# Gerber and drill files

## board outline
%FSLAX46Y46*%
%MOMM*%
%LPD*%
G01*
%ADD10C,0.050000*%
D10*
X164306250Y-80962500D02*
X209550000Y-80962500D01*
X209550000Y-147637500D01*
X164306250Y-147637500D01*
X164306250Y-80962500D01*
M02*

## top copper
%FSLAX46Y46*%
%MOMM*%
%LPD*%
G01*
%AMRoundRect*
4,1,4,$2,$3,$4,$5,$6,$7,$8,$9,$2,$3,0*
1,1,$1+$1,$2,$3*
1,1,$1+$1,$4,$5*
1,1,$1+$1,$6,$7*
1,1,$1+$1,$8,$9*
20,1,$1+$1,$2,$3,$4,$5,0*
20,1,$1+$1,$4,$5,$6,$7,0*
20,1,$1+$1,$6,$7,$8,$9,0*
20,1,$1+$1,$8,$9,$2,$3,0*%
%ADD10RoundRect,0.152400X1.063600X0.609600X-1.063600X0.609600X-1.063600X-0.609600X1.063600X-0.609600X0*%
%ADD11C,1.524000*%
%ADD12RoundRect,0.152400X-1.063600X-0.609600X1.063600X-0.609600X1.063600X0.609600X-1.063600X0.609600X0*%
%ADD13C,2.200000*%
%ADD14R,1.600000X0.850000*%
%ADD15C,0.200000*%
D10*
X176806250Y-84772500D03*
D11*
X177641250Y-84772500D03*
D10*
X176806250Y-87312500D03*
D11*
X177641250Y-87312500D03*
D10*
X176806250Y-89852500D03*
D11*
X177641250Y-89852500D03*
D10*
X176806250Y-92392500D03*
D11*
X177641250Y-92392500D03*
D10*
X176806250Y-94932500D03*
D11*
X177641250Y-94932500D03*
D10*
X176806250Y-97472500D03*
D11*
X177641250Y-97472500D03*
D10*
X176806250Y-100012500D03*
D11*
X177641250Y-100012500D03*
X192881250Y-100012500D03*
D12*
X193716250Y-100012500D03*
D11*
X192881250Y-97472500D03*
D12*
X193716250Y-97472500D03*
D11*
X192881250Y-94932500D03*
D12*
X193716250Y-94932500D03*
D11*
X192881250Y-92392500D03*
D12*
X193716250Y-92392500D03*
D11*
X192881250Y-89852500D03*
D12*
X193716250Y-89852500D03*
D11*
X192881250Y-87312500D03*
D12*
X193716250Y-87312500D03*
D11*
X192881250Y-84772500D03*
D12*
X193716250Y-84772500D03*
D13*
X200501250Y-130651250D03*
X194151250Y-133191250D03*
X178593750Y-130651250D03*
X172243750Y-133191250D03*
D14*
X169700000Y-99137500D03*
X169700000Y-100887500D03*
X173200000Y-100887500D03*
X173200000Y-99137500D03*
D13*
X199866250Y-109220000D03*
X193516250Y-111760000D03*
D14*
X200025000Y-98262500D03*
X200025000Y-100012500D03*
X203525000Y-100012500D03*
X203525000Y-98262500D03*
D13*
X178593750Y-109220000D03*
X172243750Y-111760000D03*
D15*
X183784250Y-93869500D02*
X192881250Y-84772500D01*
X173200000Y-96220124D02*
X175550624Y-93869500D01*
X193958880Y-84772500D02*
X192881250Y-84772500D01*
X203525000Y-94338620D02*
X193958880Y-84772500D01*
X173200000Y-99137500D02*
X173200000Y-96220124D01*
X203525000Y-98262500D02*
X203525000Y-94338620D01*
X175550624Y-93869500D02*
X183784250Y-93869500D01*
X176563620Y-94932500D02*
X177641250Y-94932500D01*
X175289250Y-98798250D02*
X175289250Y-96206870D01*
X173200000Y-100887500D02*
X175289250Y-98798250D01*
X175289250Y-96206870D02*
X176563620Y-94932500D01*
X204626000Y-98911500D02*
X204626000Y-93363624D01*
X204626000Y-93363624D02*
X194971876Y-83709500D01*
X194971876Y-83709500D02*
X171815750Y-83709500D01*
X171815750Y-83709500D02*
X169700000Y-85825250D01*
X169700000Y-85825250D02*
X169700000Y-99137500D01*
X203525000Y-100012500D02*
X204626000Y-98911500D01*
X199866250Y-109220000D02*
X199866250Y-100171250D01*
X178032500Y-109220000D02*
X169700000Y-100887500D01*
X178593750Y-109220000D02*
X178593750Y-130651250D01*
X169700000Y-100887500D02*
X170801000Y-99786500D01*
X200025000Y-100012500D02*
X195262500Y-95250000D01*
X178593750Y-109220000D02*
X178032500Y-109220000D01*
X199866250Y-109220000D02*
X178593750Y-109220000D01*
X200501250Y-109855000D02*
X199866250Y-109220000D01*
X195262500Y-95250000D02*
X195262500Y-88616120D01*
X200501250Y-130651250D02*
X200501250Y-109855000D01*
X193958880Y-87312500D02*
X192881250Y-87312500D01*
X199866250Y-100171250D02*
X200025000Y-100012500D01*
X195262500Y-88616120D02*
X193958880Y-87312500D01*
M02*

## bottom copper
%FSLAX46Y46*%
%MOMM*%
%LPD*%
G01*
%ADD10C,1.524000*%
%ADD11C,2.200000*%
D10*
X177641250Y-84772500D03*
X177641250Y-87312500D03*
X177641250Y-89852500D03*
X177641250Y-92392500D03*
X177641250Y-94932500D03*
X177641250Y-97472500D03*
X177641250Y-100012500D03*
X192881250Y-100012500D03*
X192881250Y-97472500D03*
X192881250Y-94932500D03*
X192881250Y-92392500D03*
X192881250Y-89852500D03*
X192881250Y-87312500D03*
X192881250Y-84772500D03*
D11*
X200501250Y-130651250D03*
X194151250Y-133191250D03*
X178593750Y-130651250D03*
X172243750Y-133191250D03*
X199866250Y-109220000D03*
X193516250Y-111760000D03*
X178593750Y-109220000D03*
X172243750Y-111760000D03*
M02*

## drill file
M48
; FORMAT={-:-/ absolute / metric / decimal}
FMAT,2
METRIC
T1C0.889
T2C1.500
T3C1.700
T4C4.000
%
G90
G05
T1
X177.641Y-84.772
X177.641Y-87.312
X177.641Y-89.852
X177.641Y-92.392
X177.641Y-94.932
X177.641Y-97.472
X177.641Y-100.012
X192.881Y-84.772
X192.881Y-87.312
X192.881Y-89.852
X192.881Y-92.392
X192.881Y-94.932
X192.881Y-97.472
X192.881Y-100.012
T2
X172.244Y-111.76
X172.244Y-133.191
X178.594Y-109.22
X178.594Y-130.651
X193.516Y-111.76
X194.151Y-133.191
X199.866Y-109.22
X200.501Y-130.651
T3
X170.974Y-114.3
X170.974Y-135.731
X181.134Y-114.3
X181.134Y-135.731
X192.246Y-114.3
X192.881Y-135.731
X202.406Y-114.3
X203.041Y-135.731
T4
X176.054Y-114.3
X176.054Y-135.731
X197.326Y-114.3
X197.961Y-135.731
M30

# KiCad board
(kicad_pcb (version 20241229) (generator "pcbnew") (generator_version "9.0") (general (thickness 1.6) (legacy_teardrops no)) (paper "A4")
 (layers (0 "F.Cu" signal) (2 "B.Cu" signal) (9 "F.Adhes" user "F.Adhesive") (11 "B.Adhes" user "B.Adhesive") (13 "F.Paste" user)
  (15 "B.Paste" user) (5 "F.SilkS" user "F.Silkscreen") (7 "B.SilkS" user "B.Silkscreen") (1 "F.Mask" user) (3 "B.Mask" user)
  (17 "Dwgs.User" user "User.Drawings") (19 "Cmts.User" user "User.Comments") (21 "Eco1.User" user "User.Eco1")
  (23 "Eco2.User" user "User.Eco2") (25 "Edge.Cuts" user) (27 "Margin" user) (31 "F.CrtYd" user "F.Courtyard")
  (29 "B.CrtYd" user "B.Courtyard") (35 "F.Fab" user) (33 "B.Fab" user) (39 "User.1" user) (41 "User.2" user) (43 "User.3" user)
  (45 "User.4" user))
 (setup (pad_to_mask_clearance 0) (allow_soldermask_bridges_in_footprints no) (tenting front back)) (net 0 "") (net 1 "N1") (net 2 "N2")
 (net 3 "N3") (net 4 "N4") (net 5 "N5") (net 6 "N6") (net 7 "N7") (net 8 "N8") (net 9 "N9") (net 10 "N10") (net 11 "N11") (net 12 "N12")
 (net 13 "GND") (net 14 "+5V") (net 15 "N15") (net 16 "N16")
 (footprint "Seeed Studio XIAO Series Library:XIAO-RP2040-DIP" (layer "F.Cu") (at 185.26125 92.3925)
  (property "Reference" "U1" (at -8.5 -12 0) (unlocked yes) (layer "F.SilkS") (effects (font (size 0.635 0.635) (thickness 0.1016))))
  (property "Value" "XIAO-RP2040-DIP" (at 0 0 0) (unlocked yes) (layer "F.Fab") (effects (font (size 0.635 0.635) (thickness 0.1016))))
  (pad "1" smd roundrect (at -8.455 -7.62 180) (size 2.432 1.524) (layers "F.Cu" "F.Mask") (roundrect_rratio 0.1) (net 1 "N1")
   (thermal_bridge_angle 45))
  (pad "1" thru_hole circle (at -7.62 -7.62 180) (size 1.524 1.524) (drill 0.889) (layers "*.Cu" "*.Mask") (remove_unused_layers no)
   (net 1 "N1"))
  (pad "2" smd roundrect (at -8.455 -5.08 180) (size 2.432 1.524) (layers "F.Cu" "F.Mask") (roundrect_rratio 0.1) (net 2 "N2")
   (thermal_bridge_angle 45))
  (pad "2" thru_hole circle (at -7.62 -5.08 180) (size 1.524 1.524) (drill 0.889) (layers "*.Cu" "*.Mask") (remove_unused_layers no)
   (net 2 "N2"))
  (pad "3" smd roundrect (at -8.455 -2.54 180) (size 2.432 1.524) (layers "F.Cu" "F.Mask") (roundrect_rratio 0.1) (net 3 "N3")
   (thermal_bridge_angle 45))
  (pad "3" thru_hole circle (at -7.62 -2.54 180) (size 1.524 1.524) (drill 0.889) (layers "*.Cu" "*.Mask") (remove_unused_layers no)
   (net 3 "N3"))
  (pad "4" smd roundrect (at -8.455 0 180) (size 2.432 1.524) (layers "F.Cu" "F.Mask") (roundrect_rratio 0.1) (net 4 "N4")
   (thermal_bridge_angle 45))
  (pad "4" thru_hole circle (at -7.62 0 180) (size 1.524 1.524) (drill 0.889) (layers "*.Cu" "*.Mask") (remove_unused_layers no)
   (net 4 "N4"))
  (pad "5" smd roundrect (at -8.455 2.54 180) (size 2.432 1.524) (layers "F.Cu" "F.Mask") (roundrect_rratio 0.1) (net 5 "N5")
   (thermal_bridge_angle 45))
  (pad "5" thru_hole circle (at -7.62 2.54 180) (size 1.524 1.524) (drill 0.889) (layers "*.Cu" "*.Mask") (remove_unused_layers no)
   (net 5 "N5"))
  (pad "6" smd roundrect (at -8.455 5.08 180) (size 2.432 1.524) (layers "F.Cu" "F.Mask") (roundrect_rratio 0.1) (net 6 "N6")
   (thermal_bridge_angle 45))
  (pad "6" thru_hole circle (at -7.62 5.08 180) (size 1.524 1.524) (drill 0.889) (layers "*.Cu" "*.Mask") (remove_unused_layers no)
   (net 6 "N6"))
  (pad "7" smd roundrect (at -8.455 7.62 180) (size 2.432 1.524) (layers "F.Cu" "F.Mask") (roundrect_rratio 0.1) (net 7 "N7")
   (thermal_bridge_angle 45))
  (pad "7" thru_hole circle (at -7.62 7.62 180) (size 1.524 1.524) (drill 0.889) (layers "*.Cu" "*.Mask") (remove_unused_layers no)
   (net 7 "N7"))
  (pad "8" thru_hole circle (at 7.62 7.62) (size 1.524 1.524) (drill 0.889) (layers "*.Cu" "*.Mask") (remove_unused_layers no) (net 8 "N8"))
  (pad "8" smd roundrect (at 8.455 7.62) (size 2.432 1.524) (layers "F.Cu" "F.Mask") (roundrect_rratio 0.1) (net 8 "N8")
   (thermal_bridge_angle 45))
  (pad "9" thru_hole circle (at 7.62 5.08) (size 1.524 1.524) (drill 0.889) (layers "*.Cu" "*.Mask") (remove_unused_layers no) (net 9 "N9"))
  (pad "9" smd roundrect (at 8.455 5.08) (size 2.432 1.524) (layers "F.Cu" "F.Mask") (roundrect_rratio 0.1) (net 9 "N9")
   (thermal_bridge_angle 45))
  (pad "10" thru_hole circle (at 7.62 2.54) (size 1.524 1.524) (drill 0.889) (layers "*.Cu" "*.Mask") (remove_unused_layers no)
   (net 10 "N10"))
  (pad "10" smd roundrect (at 8.455 2.54) (size 2.432 1.524) (layers "F.Cu" "F.Mask") (roundrect_rratio 0.1) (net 10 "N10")
   (thermal_bridge_angle 45))
  (pad "11" thru_hole circle (at 7.62 0) (size 1.524 1.524) (drill 0.889) (layers "*.Cu" "*.Mask") (remove_unused_layers no) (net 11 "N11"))
  (pad "11" smd roundrect (at 8.455 0) (size 2.432 1.524) (layers "F.Cu" "F.Mask") (roundrect_rratio 0.1) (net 11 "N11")
   (thermal_bridge_angle 45))
  (pad "12" thru_hole circle (at 7.62 -2.54) (size 1.524 1.524) (drill 0.889) (layers "*.Cu" "*.Mask") (remove_unused_layers no)
   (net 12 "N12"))
  (pad "12" smd roundrect (at 8.455 -2.54) (size 2.432 1.524) (layers "F.Cu" "F.Mask") (roundrect_rratio 0.1) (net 12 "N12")
   (thermal_bridge_angle 45))
  (pad "13" thru_hole circle (at 7.62 -5.08) (size 1.524 1.524) (drill 0.889) (layers "*.Cu" "*.Mask") (remove_unused_layers no)
   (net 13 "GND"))
  (pad "13" smd roundrect (at 8.455 -5.08) (size 2.432 1.524) (layers "F.Cu" "F.Mask") (roundrect_rratio 0.1) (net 13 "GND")
   (thermal_bridge_angle 45))
  (pad "14" thru_hole circle (at 7.62 -7.62) (size 1.524 1.524) (drill 0.889) (layers "*.Cu" "*.Mask") (remove_unused_layers no)
   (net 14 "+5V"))
  (pad "14" smd roundrect (at 8.455 -7.62) (size 2.432 1.524) (layers "F.Cu" "F.Mask") (roundrect_rratio 0.1) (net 14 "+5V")
   (thermal_bridge_angle 45)))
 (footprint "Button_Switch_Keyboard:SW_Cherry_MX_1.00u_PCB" (layer "F.Cu") (at 200.50125 130.65125)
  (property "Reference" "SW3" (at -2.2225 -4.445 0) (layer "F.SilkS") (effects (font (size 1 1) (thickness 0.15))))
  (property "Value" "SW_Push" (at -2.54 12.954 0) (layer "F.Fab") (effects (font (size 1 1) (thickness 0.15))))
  (pad "" np_thru_hole circle (at -7.62 5.08) (size 1.7 1.7) (drill 1.7) (layers "*.Cu" "*.Mask"))
  (pad "" np_thru_hole circle (at -2.54 5.08) (size 4 4) (drill 4) (layers "*.Cu" "*.Mask"))
  (pad "" np_thru_hole circle (at 2.54 5.08) (size 1.7 1.7) (drill 1.7) (layers "*.Cu" "*.Mask"))
  (pad "1" thru_hole circle (at 0 0) (size 2.2 2.2) (drill 1.5) (layers "*.Cu" "*.Mask") (remove_unused_layers no) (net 13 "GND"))
  (pad "2" thru_hole circle (at -6.35 2.54) (size 2.2 2.2) (drill 1.5) (layers "*.Cu" "*.Mask") (remove_unused_layers no) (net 11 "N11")))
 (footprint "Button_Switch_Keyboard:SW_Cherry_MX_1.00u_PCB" (layer "F.Cu") (at 178.59375 130.65125)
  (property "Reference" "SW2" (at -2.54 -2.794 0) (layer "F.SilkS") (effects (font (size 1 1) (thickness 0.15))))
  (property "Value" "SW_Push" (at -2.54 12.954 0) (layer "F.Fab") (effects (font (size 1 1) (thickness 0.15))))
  (pad "" np_thru_hole circle (at -7.62 5.08) (size 1.7 1.7) (drill 1.7) (layers "*.Cu" "*.Mask"))
  (pad "" np_thru_hole circle (at -2.54 5.08) (size 4 4) (drill 4) (layers "*.Cu" "*.Mask"))
  (pad "" np_thru_hole circle (at 2.54 5.08) (size 1.7 1.7) (drill 1.7) (layers "*.Cu" "*.Mask"))
  (pad "1" thru_hole circle (at 0 0) (size 2.2 2.2) (drill 1.5) (layers "*.Cu" "*.Mask") (remove_unused_layers no) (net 13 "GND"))
  (pad "2" thru_hole circle (at -6.35 2.54) (size 2.2 2.2) (drill 1.5) (layers "*.Cu" "*.Mask") (remove_unused_layers no) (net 10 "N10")))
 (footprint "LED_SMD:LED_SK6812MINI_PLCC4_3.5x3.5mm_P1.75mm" (layer "F.Cu") (at 171.45 100.0125)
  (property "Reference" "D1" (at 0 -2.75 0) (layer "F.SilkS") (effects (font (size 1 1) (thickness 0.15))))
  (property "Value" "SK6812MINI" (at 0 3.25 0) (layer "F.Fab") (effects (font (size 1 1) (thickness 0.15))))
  (pad "1" smd rect (at -1.75 -0.875) (size 1.6 0.85) (layers "F.Cu" "F.Mask" "F.Paste") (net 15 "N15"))
  (pad "2" smd rect (at -1.75 0.875) (size 1.6 0.85) (layers "F.Cu" "F.Mask" "F.Paste") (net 13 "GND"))
  (pad "3" smd rect (at 1.75 0.875) (size 1.6 0.85) (layers "F.Cu" "F.Mask" "F.Paste") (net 5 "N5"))
  (pad "4" smd rect (at 1.75 -0.875) (size 1.6 0.85) (layers "F.Cu" "F.Mask" "F.Paste") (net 14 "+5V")))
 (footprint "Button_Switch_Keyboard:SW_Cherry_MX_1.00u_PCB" (layer "F.Cu") (at 199.86625 109.22)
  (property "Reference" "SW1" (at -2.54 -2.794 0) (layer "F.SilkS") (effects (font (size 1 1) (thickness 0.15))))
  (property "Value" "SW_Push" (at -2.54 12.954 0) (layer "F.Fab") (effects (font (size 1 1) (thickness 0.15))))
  (pad "" np_thru_hole circle (at -7.62 5.08) (size 1.7 1.7) (drill 1.7) (layers "*.Cu" "*.Mask"))
  (pad "" np_thru_hole circle (at -2.54 5.08) (size 4 4) (drill 4) (layers "*.Cu" "*.Mask"))
  (pad "" np_thru_hole circle (at 2.54 5.08) (size 1.7 1.7) (drill 1.7) (layers "*.Cu" "*.Mask"))
  (pad "1" thru_hole circle (at 0 0) (size 2.2 2.2) (drill 1.5) (layers "*.Cu" "*.Mask") (remove_unused_layers no) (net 13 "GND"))
  (pad "2" thru_hole circle (at -6.35 2.54) (size 2.2 2.2) (drill 1.5) (layers "*.Cu" "*.Mask") (remove_unused_layers no) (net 9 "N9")))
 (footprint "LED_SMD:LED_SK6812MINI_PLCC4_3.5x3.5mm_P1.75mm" (layer "F.Cu") (at 201.775 99.1375)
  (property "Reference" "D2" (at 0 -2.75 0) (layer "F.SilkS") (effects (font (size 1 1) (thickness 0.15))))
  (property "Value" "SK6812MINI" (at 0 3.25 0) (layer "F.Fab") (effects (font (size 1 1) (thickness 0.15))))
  (pad "1" smd rect (at -1.75 -0.875) (size 1.6 0.85) (layers "F.Cu" "F.Mask" "F.Paste") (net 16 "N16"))
  (pad "2" smd rect (at -1.75 0.875) (size 1.6 0.85) (layers "F.Cu" "F.Mask" "F.Paste") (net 13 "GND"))
  (pad "3" smd rect (at 1.75 0.875) (size 1.6 0.85) (layers "F.Cu" "F.Mask" "F.Paste") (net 15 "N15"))
  (pad "4" smd rect (at 1.75 -0.875) (size 1.6 0.85) (layers "F.Cu" "F.Mask" "F.Paste") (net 14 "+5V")))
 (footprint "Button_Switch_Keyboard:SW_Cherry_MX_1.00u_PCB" (layer "F.Cu") (at 178.59375 109.22)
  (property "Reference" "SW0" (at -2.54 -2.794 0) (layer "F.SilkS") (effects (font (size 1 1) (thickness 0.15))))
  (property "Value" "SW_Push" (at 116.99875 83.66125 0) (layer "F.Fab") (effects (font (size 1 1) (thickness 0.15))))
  (pad "" np_thru_hole circle (at -7.62 5.08) (size 1.7 1.7) (drill 1.7) (layers "*.Cu" "*.Mask"))
  (pad "" np_thru_hole circle (at -2.54 5.08) (size 4 4) (drill 4) (layers "*.Cu" "*.Mask"))
  (pad "" np_thru_hole circle (at 2.54 5.08) (size 1.7 1.7) (drill 1.7) (layers "*.Cu" "*.Mask"))
  (pad "1" thru_hole circle (at 0 0) (size 2.2 2.2) (drill 1.5) (layers "*.Cu" "*.Mask") (remove_unused_layers no) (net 13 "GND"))
  (pad "2" thru_hole circle (at -6.35 2.54) (size 2.2 2.2) (drill 1.5) (layers "*.Cu" "*.Mask") (remove_unused_layers no) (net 8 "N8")))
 (gr_rect (start 164.30625 80.9625) (end 209.55 147.6375) (stroke (width 0.05) (type default)) (fill no) (layer "Edge.Cuts"))
 (segment (start 183.78425 93.8695) (end 192.88125 84.7725) (width 0.2) (layer "F.Cu") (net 14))
 (segment (start 173.2 96.220124) (end 175.550624 93.8695) (width 0.2) (layer "F.Cu") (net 14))
 (segment (start 193.95888 84.7725) (end 192.88125 84.7725) (width 0.2) (layer "F.Cu") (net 14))
 (segment (start 203.525 94.33862) (end 193.95888 84.7725) (width 0.2) (layer "F.Cu") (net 14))
 (segment (start 173.2 99.1375) (end 173.2 96.220124) (width 0.2) (layer "F.Cu") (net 14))
 (segment (start 203.525 98.2625) (end 203.525 94.33862) (width 0.2) (layer "F.Cu") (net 14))
 (segment (start 175.550624 93.8695) (end 183.78425 93.8695) (width 0.2) (layer "F.Cu") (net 14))
 (segment (start 176.56362 94.9325) (end 177.64125 94.9325) (width 0.2) (layer "F.Cu") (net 5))
 (segment (start 175.28925 98.79825) (end 175.28925 96.20687) (width 0.2) (layer "F.Cu") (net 5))
 (segment (start 173.2 100.8875) (end 175.28925 98.79825) (width 0.2) (layer "F.Cu") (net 5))
 (segment (start 175.28925 96.20687) (end 176.56362 94.9325) (width 0.2) (layer "F.Cu") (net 5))
 (segment (start 204.626 98.9115) (end 204.626 93.363624) (width 0.2) (layer "F.Cu") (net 15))
 (segment (start 204.626 93.363624) (end 194.971876 83.7095) (width 0.2) (layer "F.Cu") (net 15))
 (segment (start 194.971876 83.7095) (end 171.81575 83.7095) (width 0.2) (layer "F.Cu") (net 15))
 (segment (start 171.81575 83.7095) (end 169.7 85.82525) (width 0.2) (layer "F.Cu") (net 15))
 (segment (start 169.7 85.82525) (end 169.7 99.1375) (width 0.2) (layer "F.Cu") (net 15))
 (segment (start 203.525 100.0125) (end 204.626 98.9115) (width 0.2) (layer "F.Cu") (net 15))
 (segment (start 199.86625 109.22) (end 199.86625 100.17125) (width 0.2) (layer "F.Cu") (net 13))
 (segment (start 178.0325 109.22) (end 169.7 100.8875) (width 0.2) (layer "F.Cu") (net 13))
 (segment (start 178.59375 109.22) (end 178.59375 130.65125) (width 0.2) (layer "F.Cu") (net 13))
 (segment (start 169.7 100.8875) (end 170.801 99.7865) (width 0.2) (layer "F.Cu") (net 13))
 (segment (start 200.025 100.0125) (end 195.2625 95.25) (width 0.2) (layer "F.Cu") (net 13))
 (segment (start 178.59375 109.22) (end 178.0325 109.22) (width 0.2) (layer "F.Cu") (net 13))
 (segment (start 199.86625 109.22) (end 178.59375 109.22) (width 0.2) (layer "F.Cu") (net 13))
 (segment (start 200.50125 109.855) (end 199.86625 109.22) (width 0.2) (layer "F.Cu") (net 13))
 (segment (start 195.2625 95.25) (end 195.2625 88.61612) (width 0.2) (layer "F.Cu") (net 13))
 (segment (start 200.50125 130.65125) (end 200.50125 109.855) (width 0.2) (layer "F.Cu") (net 13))
 (segment (start 193.95888 87.3125) (end 192.88125 87.3125) (width 0.2) (layer "F.Cu") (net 13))
 (segment (start 199.86625 100.17125) (end 200.025 100.0125) (width 0.2) (layer "F.Cu") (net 13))
 (segment (start 195.2625 88.61612) (end 193.95888 87.3125) (width 0.2) (layer "F.Cu") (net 13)))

